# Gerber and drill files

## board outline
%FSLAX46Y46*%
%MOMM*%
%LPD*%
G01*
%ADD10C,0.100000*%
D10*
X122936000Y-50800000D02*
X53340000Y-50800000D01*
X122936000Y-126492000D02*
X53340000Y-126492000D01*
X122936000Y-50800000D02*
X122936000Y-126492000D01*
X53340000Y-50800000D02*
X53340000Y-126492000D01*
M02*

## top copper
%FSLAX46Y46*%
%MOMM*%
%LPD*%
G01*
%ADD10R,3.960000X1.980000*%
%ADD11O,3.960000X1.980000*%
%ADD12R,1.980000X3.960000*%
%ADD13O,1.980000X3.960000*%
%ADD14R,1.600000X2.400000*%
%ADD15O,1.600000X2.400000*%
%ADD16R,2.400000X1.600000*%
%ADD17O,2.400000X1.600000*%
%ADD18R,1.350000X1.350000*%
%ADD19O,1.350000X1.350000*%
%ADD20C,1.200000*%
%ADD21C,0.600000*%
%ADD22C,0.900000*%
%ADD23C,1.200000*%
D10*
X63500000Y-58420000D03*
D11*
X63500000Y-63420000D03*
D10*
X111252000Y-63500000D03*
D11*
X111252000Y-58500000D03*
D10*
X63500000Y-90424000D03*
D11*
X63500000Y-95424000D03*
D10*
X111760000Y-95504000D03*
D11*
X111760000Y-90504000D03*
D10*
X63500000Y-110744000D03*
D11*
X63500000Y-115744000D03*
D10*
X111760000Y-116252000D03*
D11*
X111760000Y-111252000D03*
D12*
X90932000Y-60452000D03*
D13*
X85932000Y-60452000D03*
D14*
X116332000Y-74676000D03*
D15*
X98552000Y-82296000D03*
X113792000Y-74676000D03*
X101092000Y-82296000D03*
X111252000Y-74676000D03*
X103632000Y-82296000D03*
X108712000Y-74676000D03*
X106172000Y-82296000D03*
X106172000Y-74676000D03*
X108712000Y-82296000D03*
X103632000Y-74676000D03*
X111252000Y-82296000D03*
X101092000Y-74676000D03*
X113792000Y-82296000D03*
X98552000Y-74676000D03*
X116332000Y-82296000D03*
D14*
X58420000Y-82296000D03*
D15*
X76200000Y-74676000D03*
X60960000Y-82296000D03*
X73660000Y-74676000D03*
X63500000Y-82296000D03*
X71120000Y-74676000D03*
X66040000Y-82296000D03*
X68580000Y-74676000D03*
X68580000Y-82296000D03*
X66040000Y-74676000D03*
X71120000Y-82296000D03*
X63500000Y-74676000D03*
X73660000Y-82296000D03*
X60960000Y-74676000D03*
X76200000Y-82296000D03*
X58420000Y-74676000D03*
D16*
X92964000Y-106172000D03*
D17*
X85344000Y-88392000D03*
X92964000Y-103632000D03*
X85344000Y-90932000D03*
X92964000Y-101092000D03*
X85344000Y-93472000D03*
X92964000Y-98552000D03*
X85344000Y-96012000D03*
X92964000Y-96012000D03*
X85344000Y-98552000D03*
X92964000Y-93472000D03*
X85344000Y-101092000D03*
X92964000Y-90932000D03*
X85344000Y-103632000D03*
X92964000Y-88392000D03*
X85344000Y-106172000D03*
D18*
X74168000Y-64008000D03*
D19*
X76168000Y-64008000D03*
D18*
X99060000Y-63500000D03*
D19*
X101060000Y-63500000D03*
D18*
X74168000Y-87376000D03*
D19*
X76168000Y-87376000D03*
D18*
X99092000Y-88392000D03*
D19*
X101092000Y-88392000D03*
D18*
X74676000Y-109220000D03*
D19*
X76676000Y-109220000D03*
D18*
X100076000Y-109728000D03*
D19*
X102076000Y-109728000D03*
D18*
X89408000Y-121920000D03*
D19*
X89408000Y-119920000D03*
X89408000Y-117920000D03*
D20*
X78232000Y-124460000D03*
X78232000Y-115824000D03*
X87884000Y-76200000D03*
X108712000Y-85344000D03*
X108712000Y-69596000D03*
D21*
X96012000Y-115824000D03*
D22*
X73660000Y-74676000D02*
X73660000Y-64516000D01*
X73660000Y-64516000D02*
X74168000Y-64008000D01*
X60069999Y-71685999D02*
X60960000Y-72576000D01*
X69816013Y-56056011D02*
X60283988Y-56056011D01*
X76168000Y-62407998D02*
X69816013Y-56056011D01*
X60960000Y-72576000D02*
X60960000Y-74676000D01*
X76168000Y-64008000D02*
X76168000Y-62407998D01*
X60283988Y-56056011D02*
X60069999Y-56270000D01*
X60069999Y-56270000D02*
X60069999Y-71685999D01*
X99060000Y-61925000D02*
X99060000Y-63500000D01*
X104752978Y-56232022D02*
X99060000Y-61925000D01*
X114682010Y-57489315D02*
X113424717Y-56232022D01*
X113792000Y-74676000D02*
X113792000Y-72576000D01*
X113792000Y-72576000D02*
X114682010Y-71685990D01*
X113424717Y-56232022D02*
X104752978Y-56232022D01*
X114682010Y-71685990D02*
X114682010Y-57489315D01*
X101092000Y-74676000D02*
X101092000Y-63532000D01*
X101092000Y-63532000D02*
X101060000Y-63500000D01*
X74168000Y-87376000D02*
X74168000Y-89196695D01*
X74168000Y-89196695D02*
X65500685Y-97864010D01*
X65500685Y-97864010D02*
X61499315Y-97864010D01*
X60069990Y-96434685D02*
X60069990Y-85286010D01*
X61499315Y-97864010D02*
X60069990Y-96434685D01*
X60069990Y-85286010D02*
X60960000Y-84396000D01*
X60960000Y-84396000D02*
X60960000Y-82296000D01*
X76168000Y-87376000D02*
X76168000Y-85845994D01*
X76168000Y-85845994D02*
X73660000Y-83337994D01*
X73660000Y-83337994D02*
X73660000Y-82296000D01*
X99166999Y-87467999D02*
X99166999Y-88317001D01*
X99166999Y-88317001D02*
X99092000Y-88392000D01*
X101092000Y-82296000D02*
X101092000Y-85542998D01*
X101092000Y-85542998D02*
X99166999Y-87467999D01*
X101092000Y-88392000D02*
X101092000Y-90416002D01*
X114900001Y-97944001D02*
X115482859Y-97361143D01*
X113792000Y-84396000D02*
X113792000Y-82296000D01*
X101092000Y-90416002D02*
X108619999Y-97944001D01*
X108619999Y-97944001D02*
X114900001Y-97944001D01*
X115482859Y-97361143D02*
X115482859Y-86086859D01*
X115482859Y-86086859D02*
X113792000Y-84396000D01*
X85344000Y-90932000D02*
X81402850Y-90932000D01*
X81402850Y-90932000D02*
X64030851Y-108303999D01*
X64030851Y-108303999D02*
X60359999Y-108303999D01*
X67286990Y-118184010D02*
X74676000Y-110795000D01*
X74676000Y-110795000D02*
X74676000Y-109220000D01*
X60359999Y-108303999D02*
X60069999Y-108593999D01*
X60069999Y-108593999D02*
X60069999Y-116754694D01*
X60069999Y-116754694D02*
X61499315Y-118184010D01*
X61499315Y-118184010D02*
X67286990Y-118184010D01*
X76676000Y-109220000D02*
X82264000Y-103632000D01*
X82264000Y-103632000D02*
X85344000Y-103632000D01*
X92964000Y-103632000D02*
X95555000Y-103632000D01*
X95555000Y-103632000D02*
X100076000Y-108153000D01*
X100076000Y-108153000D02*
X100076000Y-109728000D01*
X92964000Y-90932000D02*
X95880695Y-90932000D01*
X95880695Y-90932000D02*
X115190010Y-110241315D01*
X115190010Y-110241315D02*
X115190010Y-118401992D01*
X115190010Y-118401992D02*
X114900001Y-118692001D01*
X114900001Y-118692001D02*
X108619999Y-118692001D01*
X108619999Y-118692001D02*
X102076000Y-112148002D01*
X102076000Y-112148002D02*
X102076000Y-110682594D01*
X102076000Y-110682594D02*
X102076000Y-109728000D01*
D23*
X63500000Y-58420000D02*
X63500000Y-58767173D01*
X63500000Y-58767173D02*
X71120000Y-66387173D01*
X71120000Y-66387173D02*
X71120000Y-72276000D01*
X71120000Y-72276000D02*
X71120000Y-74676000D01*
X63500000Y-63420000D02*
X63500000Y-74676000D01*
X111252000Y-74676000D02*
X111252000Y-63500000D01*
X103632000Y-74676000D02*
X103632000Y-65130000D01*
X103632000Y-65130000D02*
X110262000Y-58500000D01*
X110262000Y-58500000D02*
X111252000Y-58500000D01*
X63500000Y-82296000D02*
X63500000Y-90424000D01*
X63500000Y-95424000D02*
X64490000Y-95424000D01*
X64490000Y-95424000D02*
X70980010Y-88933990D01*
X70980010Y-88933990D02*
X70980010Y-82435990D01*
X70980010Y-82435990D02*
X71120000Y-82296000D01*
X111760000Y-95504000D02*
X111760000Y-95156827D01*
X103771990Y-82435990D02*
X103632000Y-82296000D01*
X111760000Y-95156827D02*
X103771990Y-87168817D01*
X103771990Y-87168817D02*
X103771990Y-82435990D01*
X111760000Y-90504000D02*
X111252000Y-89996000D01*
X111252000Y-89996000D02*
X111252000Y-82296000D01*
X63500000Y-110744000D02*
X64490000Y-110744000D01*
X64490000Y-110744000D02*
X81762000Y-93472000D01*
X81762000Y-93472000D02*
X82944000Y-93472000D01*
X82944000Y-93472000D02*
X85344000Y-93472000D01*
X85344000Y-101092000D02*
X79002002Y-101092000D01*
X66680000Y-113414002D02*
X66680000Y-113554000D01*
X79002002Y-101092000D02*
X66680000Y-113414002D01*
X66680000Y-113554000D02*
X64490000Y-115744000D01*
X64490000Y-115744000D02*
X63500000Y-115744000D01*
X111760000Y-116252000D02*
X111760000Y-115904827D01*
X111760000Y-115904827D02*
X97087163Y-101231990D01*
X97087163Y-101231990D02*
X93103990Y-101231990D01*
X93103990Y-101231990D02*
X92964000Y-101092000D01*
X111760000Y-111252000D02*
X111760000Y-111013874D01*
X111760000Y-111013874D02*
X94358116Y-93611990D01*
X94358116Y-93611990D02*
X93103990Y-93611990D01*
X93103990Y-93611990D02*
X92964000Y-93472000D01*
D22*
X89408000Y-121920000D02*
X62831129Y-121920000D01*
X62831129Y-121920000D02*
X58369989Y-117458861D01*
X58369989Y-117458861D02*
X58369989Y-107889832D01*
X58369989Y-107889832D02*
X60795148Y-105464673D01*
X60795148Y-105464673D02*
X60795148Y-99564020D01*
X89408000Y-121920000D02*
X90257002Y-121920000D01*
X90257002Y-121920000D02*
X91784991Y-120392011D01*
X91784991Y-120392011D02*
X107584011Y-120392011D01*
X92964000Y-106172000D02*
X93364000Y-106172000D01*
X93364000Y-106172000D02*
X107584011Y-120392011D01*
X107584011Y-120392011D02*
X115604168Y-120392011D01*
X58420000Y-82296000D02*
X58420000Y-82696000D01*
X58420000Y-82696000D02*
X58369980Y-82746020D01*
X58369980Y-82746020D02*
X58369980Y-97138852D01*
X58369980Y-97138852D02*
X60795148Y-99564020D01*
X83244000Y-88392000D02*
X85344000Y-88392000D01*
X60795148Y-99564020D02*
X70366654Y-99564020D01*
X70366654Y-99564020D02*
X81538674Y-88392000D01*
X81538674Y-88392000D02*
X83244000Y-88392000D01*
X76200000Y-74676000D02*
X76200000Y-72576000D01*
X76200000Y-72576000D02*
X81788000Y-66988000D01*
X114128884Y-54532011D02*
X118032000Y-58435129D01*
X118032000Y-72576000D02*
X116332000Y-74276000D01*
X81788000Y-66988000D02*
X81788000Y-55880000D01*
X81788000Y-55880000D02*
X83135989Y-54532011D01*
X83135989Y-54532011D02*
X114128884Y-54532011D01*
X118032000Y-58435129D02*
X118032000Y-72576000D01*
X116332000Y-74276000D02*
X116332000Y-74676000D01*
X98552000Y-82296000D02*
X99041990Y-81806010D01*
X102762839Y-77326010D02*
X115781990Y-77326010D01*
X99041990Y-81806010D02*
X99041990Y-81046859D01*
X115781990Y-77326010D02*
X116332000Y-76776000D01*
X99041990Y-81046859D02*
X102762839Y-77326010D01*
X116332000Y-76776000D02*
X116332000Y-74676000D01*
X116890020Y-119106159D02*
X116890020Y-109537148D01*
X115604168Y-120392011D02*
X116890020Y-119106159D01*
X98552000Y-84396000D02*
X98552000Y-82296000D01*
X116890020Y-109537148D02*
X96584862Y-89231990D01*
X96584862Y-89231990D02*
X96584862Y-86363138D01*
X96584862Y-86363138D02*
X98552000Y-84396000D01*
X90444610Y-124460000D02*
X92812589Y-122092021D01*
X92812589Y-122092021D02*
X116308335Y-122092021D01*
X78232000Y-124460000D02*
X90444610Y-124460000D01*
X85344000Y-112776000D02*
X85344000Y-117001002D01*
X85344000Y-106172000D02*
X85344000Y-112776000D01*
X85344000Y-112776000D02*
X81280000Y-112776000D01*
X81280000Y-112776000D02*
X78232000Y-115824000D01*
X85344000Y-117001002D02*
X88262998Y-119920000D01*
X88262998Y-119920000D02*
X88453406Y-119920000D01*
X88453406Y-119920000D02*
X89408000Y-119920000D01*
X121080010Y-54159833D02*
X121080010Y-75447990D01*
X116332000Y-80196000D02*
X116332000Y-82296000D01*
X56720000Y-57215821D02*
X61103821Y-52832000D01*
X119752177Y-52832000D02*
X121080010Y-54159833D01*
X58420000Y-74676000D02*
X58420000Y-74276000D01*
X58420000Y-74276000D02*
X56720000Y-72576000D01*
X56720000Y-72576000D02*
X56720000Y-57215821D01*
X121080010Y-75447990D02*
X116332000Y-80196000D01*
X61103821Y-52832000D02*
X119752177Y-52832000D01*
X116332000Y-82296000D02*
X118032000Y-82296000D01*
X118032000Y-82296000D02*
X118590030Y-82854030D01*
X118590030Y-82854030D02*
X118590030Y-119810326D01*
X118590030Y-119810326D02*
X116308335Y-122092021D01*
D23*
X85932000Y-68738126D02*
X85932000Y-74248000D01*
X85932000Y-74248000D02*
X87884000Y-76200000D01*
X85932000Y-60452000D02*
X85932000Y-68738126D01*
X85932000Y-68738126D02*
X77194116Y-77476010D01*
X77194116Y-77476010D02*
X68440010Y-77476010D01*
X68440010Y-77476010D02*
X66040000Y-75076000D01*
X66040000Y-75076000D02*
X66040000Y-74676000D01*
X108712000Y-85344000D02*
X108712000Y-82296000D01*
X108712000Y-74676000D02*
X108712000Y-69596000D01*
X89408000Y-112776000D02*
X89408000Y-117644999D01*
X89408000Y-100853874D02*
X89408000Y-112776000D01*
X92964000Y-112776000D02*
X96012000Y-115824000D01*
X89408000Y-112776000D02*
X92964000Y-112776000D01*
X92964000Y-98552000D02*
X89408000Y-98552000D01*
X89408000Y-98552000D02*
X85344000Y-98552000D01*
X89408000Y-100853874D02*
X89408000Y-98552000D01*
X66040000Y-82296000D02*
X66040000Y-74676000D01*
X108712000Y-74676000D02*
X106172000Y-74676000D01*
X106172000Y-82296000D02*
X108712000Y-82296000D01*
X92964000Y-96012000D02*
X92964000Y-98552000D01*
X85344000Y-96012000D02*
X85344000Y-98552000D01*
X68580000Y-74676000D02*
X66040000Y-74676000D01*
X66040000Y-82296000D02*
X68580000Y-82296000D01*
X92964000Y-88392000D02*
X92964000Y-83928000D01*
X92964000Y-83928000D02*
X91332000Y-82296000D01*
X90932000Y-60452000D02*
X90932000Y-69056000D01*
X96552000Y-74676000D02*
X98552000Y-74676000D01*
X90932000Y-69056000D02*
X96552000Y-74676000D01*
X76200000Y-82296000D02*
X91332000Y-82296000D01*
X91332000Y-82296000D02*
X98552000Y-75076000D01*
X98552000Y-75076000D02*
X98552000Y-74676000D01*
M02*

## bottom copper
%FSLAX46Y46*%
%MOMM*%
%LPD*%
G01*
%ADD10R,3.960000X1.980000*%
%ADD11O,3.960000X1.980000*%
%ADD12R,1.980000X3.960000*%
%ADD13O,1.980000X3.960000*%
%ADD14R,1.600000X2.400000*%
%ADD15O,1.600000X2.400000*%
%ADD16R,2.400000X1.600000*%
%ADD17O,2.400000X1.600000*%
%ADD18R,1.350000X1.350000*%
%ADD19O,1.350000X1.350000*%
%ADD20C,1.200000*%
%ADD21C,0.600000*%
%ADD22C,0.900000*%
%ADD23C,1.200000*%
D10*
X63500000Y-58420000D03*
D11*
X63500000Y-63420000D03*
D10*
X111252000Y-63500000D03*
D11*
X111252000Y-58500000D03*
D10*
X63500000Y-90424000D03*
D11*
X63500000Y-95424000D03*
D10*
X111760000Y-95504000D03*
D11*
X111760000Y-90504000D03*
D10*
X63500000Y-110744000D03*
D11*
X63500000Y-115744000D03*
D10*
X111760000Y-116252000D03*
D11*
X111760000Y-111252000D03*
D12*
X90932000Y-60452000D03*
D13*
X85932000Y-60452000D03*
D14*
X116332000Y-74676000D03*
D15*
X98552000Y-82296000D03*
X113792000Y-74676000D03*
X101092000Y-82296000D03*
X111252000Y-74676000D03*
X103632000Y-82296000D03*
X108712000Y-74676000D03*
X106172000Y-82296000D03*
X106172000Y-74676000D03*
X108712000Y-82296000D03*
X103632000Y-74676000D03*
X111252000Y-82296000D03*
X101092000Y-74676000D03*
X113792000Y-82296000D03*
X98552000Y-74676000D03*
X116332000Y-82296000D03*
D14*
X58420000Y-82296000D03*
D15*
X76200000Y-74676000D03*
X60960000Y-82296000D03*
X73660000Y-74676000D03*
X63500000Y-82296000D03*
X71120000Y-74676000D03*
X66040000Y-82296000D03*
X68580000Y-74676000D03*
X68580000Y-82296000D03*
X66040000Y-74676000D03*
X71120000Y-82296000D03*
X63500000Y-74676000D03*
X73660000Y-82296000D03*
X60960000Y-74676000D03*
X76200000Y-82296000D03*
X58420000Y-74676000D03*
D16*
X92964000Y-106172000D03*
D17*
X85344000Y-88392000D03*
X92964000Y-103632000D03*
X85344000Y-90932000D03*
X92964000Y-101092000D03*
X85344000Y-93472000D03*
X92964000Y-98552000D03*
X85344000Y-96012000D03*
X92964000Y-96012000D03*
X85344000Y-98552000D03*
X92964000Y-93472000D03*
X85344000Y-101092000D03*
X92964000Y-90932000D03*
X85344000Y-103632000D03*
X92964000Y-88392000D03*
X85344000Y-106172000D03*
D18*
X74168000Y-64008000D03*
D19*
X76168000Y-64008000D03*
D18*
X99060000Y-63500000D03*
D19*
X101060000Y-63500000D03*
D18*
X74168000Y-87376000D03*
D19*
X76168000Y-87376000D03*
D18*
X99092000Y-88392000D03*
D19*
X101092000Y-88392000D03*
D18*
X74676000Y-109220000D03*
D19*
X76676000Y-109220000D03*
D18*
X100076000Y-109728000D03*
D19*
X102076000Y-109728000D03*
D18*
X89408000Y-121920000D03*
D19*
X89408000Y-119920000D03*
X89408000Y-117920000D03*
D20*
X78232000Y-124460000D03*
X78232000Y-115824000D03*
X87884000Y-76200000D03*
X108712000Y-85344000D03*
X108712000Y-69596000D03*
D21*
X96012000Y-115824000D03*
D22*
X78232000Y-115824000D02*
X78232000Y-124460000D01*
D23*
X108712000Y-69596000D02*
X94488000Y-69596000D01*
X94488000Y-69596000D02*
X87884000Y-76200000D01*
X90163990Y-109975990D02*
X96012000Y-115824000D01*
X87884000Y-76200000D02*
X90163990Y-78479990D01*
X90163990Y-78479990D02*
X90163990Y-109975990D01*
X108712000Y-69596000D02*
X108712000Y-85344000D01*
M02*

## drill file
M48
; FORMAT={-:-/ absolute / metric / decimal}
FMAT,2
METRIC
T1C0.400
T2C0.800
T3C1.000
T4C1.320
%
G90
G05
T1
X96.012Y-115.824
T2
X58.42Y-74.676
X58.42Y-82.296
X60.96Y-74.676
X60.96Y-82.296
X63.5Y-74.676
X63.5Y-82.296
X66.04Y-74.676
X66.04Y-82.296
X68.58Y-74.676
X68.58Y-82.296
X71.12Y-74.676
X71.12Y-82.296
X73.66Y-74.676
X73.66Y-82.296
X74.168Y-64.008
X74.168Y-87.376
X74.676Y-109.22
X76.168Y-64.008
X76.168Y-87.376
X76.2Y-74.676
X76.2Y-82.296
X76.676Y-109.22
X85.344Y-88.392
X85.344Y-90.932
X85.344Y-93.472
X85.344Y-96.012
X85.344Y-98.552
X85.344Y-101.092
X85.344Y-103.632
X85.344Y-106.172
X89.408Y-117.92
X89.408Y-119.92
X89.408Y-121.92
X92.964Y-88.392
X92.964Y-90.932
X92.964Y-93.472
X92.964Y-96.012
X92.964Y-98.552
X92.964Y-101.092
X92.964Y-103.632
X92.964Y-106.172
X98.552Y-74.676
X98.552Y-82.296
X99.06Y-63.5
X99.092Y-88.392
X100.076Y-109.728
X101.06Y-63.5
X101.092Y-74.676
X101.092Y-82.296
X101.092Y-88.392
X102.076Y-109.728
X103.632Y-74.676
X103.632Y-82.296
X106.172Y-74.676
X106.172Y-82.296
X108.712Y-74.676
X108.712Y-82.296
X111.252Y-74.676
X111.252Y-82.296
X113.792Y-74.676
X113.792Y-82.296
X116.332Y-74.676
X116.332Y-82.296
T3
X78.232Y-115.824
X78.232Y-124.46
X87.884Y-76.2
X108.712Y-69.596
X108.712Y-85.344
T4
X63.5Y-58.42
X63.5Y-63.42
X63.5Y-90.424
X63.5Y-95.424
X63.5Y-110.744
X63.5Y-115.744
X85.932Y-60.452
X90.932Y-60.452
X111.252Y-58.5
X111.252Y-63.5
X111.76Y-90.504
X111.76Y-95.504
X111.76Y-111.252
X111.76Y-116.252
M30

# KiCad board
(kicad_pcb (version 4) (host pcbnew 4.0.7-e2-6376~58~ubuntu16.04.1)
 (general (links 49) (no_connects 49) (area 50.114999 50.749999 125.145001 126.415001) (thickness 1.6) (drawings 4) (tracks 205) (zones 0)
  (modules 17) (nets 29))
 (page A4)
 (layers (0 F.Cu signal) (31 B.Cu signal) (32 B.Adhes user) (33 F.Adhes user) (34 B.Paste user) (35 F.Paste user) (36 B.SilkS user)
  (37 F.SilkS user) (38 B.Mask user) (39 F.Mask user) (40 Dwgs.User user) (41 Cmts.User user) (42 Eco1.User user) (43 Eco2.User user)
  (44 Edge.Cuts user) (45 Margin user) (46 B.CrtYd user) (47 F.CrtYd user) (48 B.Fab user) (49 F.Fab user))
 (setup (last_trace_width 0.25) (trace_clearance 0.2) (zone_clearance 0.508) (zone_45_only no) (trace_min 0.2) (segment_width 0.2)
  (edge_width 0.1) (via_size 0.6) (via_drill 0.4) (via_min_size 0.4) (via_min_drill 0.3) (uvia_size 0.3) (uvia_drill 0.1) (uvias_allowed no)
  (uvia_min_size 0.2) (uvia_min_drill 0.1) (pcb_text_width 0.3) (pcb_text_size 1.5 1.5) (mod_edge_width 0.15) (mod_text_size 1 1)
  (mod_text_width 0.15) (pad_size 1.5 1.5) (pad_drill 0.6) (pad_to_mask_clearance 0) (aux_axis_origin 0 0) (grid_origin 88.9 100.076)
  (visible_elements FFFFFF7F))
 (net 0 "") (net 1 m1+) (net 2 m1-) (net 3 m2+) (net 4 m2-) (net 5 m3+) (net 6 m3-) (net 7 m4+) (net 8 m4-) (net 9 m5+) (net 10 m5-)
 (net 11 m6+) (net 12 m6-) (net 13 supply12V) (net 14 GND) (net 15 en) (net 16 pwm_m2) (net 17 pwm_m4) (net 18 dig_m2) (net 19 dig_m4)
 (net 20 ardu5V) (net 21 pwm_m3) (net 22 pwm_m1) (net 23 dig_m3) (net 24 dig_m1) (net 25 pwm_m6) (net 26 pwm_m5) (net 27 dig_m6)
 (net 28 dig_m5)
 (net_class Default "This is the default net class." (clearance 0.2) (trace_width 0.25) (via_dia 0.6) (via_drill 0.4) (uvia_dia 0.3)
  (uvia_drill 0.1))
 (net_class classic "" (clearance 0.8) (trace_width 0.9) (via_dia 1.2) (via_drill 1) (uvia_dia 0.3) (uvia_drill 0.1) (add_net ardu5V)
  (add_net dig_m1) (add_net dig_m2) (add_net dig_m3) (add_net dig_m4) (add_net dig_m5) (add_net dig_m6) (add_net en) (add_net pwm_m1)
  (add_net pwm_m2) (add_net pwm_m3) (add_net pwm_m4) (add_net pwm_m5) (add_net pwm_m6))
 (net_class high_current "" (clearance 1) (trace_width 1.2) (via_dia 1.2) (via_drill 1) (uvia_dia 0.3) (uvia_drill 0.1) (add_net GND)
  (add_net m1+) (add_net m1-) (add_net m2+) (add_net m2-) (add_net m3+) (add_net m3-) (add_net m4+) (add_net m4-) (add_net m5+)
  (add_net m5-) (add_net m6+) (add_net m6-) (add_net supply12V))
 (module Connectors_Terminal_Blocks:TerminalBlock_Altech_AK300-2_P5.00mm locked (layer F.Cu) (at 63.5 58.42 270)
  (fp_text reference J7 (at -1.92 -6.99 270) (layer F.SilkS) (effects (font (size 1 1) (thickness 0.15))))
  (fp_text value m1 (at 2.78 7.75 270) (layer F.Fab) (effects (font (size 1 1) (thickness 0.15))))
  (pad 1 thru_hole rect (at 0 0 270) (size 1.98 3.96) (drill 1.32) (layers *.Cu *.Mask) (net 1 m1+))
  (pad 2 thru_hole oval (at 5 0 270) (size 1.98 3.96) (drill 1.32) (layers *.Cu *.Mask) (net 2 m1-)))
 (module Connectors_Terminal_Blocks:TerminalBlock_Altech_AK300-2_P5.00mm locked (layer F.Cu) (at 111.252 63.5 90)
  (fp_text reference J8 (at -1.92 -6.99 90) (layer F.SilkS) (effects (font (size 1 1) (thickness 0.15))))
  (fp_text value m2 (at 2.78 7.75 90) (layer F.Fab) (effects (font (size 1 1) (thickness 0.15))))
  (pad 1 thru_hole rect (at 0 0 90) (size 1.98 3.96) (drill 1.32) (layers *.Cu *.Mask) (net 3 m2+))
  (pad 2 thru_hole oval (at 5 0 90) (size 1.98 3.96) (drill 1.32) (layers *.Cu *.Mask) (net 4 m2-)))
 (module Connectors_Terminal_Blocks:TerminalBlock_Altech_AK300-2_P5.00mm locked (layer F.Cu) (at 63.5 90.424 270)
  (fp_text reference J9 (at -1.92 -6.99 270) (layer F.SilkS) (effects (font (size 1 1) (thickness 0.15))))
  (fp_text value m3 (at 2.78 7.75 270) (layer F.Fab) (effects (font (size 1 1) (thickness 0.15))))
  (pad 1 thru_hole rect (at 0 0 270) (size 1.98 3.96) (drill 1.32) (layers *.Cu *.Mask) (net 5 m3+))
  (pad 2 thru_hole oval (at 5 0 270) (size 1.98 3.96) (drill 1.32) (layers *.Cu *.Mask) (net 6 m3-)))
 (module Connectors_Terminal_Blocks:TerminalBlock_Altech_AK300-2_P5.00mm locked (layer F.Cu) (at 111.76 95.504 90)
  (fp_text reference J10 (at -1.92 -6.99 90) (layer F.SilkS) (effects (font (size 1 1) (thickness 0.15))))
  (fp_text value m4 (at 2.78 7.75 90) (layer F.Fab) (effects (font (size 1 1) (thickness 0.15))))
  (pad 1 thru_hole rect (at 0 0 90) (size 1.98 3.96) (drill 1.32) (layers *.Cu *.Mask) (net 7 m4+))
  (pad 2 thru_hole oval (at 5 0 90) (size 1.98 3.96) (drill 1.32) (layers *.Cu *.Mask) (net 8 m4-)))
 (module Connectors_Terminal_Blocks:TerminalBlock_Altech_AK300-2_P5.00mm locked (layer F.Cu) (at 63.5 110.744 270)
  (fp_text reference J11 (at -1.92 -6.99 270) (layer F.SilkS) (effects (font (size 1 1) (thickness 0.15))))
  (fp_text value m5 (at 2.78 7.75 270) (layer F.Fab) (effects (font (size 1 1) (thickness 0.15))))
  (pad 1 thru_hole rect (at 0 0 270) (size 1.98 3.96) (drill 1.32) (layers *.Cu *.Mask) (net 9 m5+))
  (pad 2 thru_hole oval (at 5 0 270) (size 1.98 3.96) (drill 1.32) (layers *.Cu *.Mask) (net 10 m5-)))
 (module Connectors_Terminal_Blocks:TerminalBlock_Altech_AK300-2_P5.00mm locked (layer F.Cu) (at 111.76 116.252 90)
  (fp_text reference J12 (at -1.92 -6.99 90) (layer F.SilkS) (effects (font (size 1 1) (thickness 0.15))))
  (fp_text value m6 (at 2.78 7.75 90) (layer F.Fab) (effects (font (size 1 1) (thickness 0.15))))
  (pad 1 thru_hole rect (at 0 0 90) (size 1.98 3.96) (drill 1.32) (layers *.Cu *.Mask) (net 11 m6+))
  (pad 2 thru_hole oval (at 5 0 90) (size 1.98 3.96) (drill 1.32) (layers *.Cu *.Mask) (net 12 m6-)))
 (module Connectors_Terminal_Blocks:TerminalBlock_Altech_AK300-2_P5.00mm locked (layer F.Cu) (at 90.932 60.452 180)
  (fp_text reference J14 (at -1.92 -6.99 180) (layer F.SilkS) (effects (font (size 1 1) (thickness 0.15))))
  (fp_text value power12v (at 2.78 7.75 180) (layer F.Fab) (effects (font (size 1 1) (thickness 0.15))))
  (pad 1 thru_hole rect (at 0 0 180) (size 1.98 3.96) (drill 1.32) (layers *.Cu *.Mask) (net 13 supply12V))
  (pad 2 thru_hole oval (at 5 0 180) (size 1.98 3.96) (drill 1.32) (layers *.Cu *.Mask) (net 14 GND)))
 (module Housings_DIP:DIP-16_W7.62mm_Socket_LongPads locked (layer F.Cu) (at 116.332 74.676 270)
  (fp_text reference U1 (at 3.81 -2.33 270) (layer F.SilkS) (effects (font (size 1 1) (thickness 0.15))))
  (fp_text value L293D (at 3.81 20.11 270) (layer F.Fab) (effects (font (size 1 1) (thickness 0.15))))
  (pad 1 thru_hole rect (at 0 0 270) (size 2.4 1.6) (drill 0.8) (layers *.Cu *.Mask) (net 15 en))
  (pad 9 thru_hole oval (at 7.62 17.78 270) (size 2.4 1.6) (drill 0.8) (layers *.Cu *.Mask) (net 15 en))
  (pad 2 thru_hole oval (at 0 2.54 270) (size 2.4 1.6) (drill 0.8) (layers *.Cu *.Mask) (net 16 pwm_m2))
  (pad 10 thru_hole oval (at 7.62 15.24 270) (size 2.4 1.6) (drill 0.8) (layers *.Cu *.Mask) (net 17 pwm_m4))
  (pad 3 thru_hole oval (at 0 5.08 270) (size 2.4 1.6) (drill 0.8) (layers *.Cu *.Mask) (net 3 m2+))
  (pad 11 thru_hole oval (at 7.62 12.7 270) (size 2.4 1.6) (drill 0.8) (layers *.Cu *.Mask) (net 7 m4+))
  (pad 4 thru_hole oval (at 0 7.62 270) (size 2.4 1.6) (drill 0.8) (layers *.Cu *.Mask) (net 14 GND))
  (pad 12 thru_hole oval (at 7.62 10.16 270) (size 2.4 1.6) (drill 0.8) (layers *.Cu *.Mask) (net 14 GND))
  (pad 5 thru_hole oval (at 0 10.16 270) (size 2.4 1.6) (drill 0.8) (layers *.Cu *.Mask) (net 14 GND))
  (pad 13 thru_hole oval (at 7.62 7.62 270) (size 2.4 1.6) (drill 0.8) (layers *.Cu *.Mask) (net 14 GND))
  (pad 6 thru_hole oval (at 0 12.7 270) (size 2.4 1.6) (drill 0.8) (layers *.Cu *.Mask) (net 4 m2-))
  (pad 14 thru_hole oval (at 7.62 5.08 270) (size 2.4 1.6) (drill 0.8) (layers *.Cu *.Mask) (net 8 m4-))
  (pad 7 thru_hole oval (at 0 15.24 270) (size 2.4 1.6) (drill 0.8) (layers *.Cu *.Mask) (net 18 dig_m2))
  (pad 15 thru_hole oval (at 7.62 2.54 270) (size 2.4 1.6) (drill 0.8) (layers *.Cu *.Mask) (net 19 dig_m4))
  (pad 8 thru_hole oval (at 0 17.78 270) (size 2.4 1.6) (drill 0.8) (layers *.Cu *.Mask) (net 13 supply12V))
  (pad 16 thru_hole oval (at 7.62 0 270) (size 2.4 1.6) (drill 0.8) (layers *.Cu *.Mask) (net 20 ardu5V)))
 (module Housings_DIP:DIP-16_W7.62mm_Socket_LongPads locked (layer F.Cu) (at 58.42 82.296 90)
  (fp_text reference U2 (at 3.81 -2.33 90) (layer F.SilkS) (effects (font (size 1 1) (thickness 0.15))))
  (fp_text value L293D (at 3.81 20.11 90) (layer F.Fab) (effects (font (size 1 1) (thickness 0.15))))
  (pad 1 thru_hole rect (at 0 0 90) (size 2.4 1.6) (drill 0.8) (layers *.Cu *.Mask) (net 15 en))
  (pad 9 thru_hole oval (at 7.62 17.78 90) (size 2.4 1.6) (drill 0.8) (layers *.Cu *.Mask) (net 15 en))
  (pad 2 thru_hole oval (at 0 2.54 90) (size 2.4 1.6) (drill 0.8) (layers *.Cu *.Mask) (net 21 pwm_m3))
  (pad 10 thru_hole oval (at 7.62 15.24 90) (size 2.4 1.6) (drill 0.8) (layers *.Cu *.Mask) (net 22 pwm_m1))
  (pad 3 thru_hole oval (at 0 5.08 90) (size 2.4 1.6) (drill 0.8) (layers *.Cu *.Mask) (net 5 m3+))
  (pad 11 thru_hole oval (at 7.62 12.7 90) (size 2.4 1.6) (drill 0.8) (layers *.Cu *.Mask) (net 1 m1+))
  (pad 4 thru_hole oval (at 0 7.62 90) (size 2.4 1.6) (drill 0.8) (layers *.Cu *.Mask) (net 14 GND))
  (pad 12 thru_hole oval (at 7.62 10.16 90) (size 2.4 1.6) (drill 0.8) (layers *.Cu *.Mask) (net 14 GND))
  (pad 5 thru_hole oval (at 0 10.16 90) (size 2.4 1.6) (drill 0.8) (layers *.Cu *.Mask) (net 14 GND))
  (pad 13 thru_hole oval (at 7.62 7.62 90) (size 2.4 1.6) (drill 0.8) (layers *.Cu *.Mask) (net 14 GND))
  (pad 6 thru_hole oval (at 0 12.7 90) (size 2.4 1.6) (drill 0.8) (layers *.Cu *.Mask) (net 6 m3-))
  (pad 14 thru_hole oval (at 7.62 5.08 90) (size 2.4 1.6) (drill 0.8) (layers *.Cu *.Mask) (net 2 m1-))
  (pad 7 thru_hole oval (at 0 15.24 90) (size 2.4 1.6) (drill 0.8) (layers *.Cu *.Mask) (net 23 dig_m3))
  (pad 15 thru_hole oval (at 7.62 2.54 90) (size 2.4 1.6) (drill 0.8) (layers *.Cu *.Mask) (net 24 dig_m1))
  (pad 8 thru_hole oval (at 0 17.78 90) (size 2.4 1.6) (drill 0.8) (layers *.Cu *.Mask) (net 13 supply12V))
  (pad 16 thru_hole oval (at 7.62 0 90) (size 2.4 1.6) (drill 0.8) (layers *.Cu *.Mask) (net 20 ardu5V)))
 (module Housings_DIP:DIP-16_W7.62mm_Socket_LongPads (layer F.Cu) (at 92.964 106.172 180)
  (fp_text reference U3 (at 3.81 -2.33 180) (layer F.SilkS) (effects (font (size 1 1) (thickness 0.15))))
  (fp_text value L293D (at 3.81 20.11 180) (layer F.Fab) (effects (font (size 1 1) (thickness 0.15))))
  (pad 1 thru_hole rect (at 0 0 180) (size 2.4 1.6) (drill 0.8) (layers *.Cu *.Mask) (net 15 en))
  (pad 9 thru_hole oval (at 7.62 17.78 180) (size 2.4 1.6) (drill 0.8) (layers *.Cu *.Mask) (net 15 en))
  (pad 2 thru_hole oval (at 0 2.54 180) (size 2.4 1.6) (drill 0.8) (layers *.Cu *.Mask) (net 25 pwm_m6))
  (pad 10 thru_hole oval (at 7.62 15.24 180) (size 2.4 1.6) (drill 0.8) (layers *.Cu *.Mask) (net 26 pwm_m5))
  (pad 3 thru_hole oval (at 0 5.08 180) (size 2.4 1.6) (drill 0.8) (layers *.Cu *.Mask) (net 11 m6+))
  (pad 11 thru_hole oval (at 7.62 12.7 180) (size 2.4 1.6) (drill 0.8) (layers *.Cu *.Mask) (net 9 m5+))
  (pad 4 thru_hole oval (at 0 7.62 180) (size 2.4 1.6) (drill 0.8) (layers *.Cu *.Mask) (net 14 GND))
  (pad 12 thru_hole oval (at 7.62 10.16 180) (size 2.4 1.6) (drill 0.8) (layers *.Cu *.Mask) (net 14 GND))
  (pad 5 thru_hole oval (at 0 10.16 180) (size 2.4 1.6) (drill 0.8) (layers *.Cu *.Mask) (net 14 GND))
  (pad 13 thru_hole oval (at 7.62 7.62 180) (size 2.4 1.6) (drill 0.8) (layers *.Cu *.Mask) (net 14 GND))
  (pad 6 thru_hole oval (at 0 12.7 180) (size 2.4 1.6) (drill 0.8) (layers *.Cu *.Mask) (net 12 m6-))
  (pad 14 thru_hole oval (at 7.62 5.08 180) (size 2.4 1.6) (drill 0.8) (layers *.Cu *.Mask) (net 10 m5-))
  (pad 7 thru_hole oval (at 0 15.24 180) (size 2.4 1.6) (drill 0.8) (layers *.Cu *.Mask) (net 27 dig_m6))
  (pad 15 thru_hole oval (at 7.62 2.54 180) (size 2.4 1.6) (drill 0.8) (layers *.Cu *.Mask) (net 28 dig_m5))
  (pad 8 thru_hole oval (at 0 17.78 180) (size 2.4 1.6) (drill 0.8) (layers *.Cu *.Mask) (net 13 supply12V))
  (pad 16 thru_hole oval (at 7.62 0 180) (size 2.4 1.6) (drill 0.8) (layers *.Cu *.Mask) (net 20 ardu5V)))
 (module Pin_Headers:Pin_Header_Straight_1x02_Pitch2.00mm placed (layer F.Cu) (at 74.168 64.008 90)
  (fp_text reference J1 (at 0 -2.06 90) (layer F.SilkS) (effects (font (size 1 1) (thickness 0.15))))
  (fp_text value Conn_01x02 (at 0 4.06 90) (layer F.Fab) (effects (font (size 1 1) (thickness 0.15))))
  (pad 1 thru_hole rect (at 0 0 90) (size 1.35 1.35) (drill 0.8) (layers *.Cu *.Mask) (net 22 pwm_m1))
  (pad 2 thru_hole oval (at 0 2 90) (size 1.35 1.35) (drill 0.8) (layers *.Cu *.Mask) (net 24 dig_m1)))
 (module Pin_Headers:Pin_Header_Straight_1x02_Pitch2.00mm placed (layer F.Cu) (at 99.06 63.5 90)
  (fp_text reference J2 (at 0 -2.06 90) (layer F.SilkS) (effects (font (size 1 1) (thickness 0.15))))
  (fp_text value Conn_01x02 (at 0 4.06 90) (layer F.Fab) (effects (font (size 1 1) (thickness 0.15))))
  (pad 1 thru_hole rect (at 0 0 90) (size 1.35 1.35) (drill 0.8) (layers *.Cu *.Mask) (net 16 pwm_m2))
  (pad 2 thru_hole oval (at 0 2 90) (size 1.35 1.35) (drill 0.8) (layers *.Cu *.Mask) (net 18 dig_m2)))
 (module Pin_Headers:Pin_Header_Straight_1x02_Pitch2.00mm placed (layer F.Cu) (at 74.168 87.376 90)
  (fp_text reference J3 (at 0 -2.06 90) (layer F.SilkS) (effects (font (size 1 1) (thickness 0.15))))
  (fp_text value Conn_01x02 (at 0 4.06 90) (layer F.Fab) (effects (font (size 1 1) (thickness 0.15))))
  (pad 1 thru_hole rect (at 0 0 90) (size 1.35 1.35) (drill 0.8) (layers *.Cu *.Mask) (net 21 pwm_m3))
  (pad 2 thru_hole oval (at 0 2 90) (size 1.35 1.35) (drill 0.8) (layers *.Cu *.Mask) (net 23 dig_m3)))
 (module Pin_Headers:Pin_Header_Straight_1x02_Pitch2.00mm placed (layer F.Cu) (at 99.092 88.392 90)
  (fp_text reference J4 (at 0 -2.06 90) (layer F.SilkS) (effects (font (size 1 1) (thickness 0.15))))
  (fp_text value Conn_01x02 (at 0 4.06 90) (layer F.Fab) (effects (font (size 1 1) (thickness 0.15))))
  (pad 1 thru_hole rect (at 0 0 90) (size 1.35 1.35) (drill 0.8) (layers *.Cu *.Mask) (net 17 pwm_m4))
  (pad 2 thru_hole oval (at 0 2 90) (size 1.35 1.35) (drill 0.8) (layers *.Cu *.Mask) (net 19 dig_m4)))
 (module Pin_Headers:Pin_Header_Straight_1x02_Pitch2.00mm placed (layer F.Cu) (at 74.676 109.22 90)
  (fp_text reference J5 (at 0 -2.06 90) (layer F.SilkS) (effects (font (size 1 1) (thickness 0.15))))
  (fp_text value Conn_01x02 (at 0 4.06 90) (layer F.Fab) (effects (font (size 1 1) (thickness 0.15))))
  (pad 1 thru_hole rect (at 0 0 90) (size 1.35 1.35) (drill 0.8) (layers *.Cu *.Mask) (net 26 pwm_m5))
  (pad 2 thru_hole oval (at 0 2 90) (size 1.35 1.35) (drill 0.8) (layers *.Cu *.Mask) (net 28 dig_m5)))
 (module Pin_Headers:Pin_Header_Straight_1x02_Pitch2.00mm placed (layer F.Cu) (at 100.076 109.728 90)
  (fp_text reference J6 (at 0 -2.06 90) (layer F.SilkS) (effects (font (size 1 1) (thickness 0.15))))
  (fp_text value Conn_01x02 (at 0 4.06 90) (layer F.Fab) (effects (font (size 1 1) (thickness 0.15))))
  (pad 1 thru_hole rect (at 0 0 90) (size 1.35 1.35) (drill 0.8) (layers *.Cu *.Mask) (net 25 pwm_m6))
  (pad 2 thru_hole oval (at 0 2 90) (size 1.35 1.35) (drill 0.8) (layers *.Cu *.Mask) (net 27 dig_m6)))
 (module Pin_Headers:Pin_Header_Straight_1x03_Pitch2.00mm (layer F.Cu) (at 89.408 121.92 180)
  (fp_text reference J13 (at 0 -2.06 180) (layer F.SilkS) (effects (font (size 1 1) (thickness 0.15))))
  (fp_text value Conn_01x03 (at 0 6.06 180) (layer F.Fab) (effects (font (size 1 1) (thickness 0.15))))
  (pad 1 thru_hole rect (at 0 0 180) (size 1.35 1.35) (drill 0.8) (layers *.Cu *.Mask) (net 15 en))
  (pad 2 thru_hole oval (at 0 2 180) (size 1.35 1.35) (drill 0.8) (layers *.Cu *.Mask) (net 20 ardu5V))
  (pad 3 thru_hole oval (at 0 4 180) (size 1.35 1.35) (drill 0.8) (layers *.Cu *.Mask) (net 14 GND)))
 (gr_line (start 122.936 50.8) (end 53.34 50.8) (layer Edge.Cuts) (width 0.1))
 (gr_line (start 122.936 126.492) (end 53.34 126.492) (layer Edge.Cuts) (width 0.1))
 (gr_line (start 122.936 50.8) (end 122.936 126.492) (layer Edge.Cuts) (width 0.1))
 (gr_line (start 53.34 50.8) (end 53.34 126.492) (layer Edge.Cuts) (width 0.1))
 (segment (start 73.66 74.676) (end 73.66 64.516) (width 0.9) (layer F.Cu) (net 22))
 (segment (start 73.66 64.516) (end 74.168 64.008) (width 0.9) (layer F.Cu) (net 22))
 (segment (start 60.069999 71.685999) (end 60.96 72.576) (width 0.9) (layer F.Cu) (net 24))
 (segment (start 69.816013 56.056011) (end 60.283988 56.056011) (width 0.9) (layer F.Cu) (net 24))
 (segment (start 76.168 62.407998) (end 69.816013 56.056011) (width 0.9) (layer F.Cu) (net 24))
 (segment (start 60.96 72.576) (end 60.96 74.676) (width 0.9) (layer F.Cu) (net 24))
 (segment (start 76.168 64.008) (end 76.168 62.407998) (width 0.9) (layer F.Cu) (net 24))
 (segment (start 60.283988 56.056011) (end 60.069999 56.27) (width 0.9) (layer F.Cu) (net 24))
 (segment (start 60.069999 56.27) (end 60.069999 71.685999) (width 0.9) (layer F.Cu) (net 24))
 (segment (start 99.06 61.925) (end 99.06 63.5) (width 0.9) (layer F.Cu) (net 16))
 (segment (start 104.752978 56.232022) (end 99.06 61.925) (width 0.9) (layer F.Cu) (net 16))
 (segment (start 114.68201 57.489315) (end 113.424717 56.232022) (width 0.9) (layer F.Cu) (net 16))
 (segment (start 113.792 74.676) (end 113.792 72.576) (width 0.9) (layer F.Cu) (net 16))
 (segment (start 113.792 72.576) (end 114.68201 71.68599) (width 0.9) (layer F.Cu) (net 16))
 (segment (start 113.424717 56.232022) (end 104.752978 56.232022) (width 0.9) (layer F.Cu) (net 16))
 (segment (start 114.68201 71.68599) (end 114.68201 57.489315) (width 0.9) (layer F.Cu) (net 16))
 (segment (start 101.092 74.676) (end 101.092 63.532) (width 0.9) (layer F.Cu) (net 18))
 (segment (start 101.092 63.532) (end 101.06 63.5) (width 0.9) (layer F.Cu) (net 18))
 (segment (start 74.168 87.376) (end 74.168 89.196695) (width 0.9) (layer F.Cu) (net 21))
 (segment (start 74.168 89.196695) (end 65.500685 97.86401) (width 0.9) (layer F.Cu) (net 21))
 (segment (start 65.500685 97.86401) (end 61.499315 97.86401) (width 0.9) (layer F.Cu) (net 21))
 (segment (start 60.06999 96.434685) (end 60.06999 85.28601) (width 0.9) (layer F.Cu) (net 21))
 (segment (start 61.499315 97.86401) (end 60.06999 96.434685) (width 0.9) (layer F.Cu) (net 21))
 (segment (start 60.06999 85.28601) (end 60.96 84.396) (width 0.9) (layer F.Cu) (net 21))
 (segment (start 60.96 84.396) (end 60.96 82.296) (width 0.9) (layer F.Cu) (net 21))
 (segment (start 76.168 87.376) (end 76.168 85.845994) (width 0.9) (layer F.Cu) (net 23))
 (segment (start 76.168 85.845994) (end 73.66 83.337994) (width 0.9) (layer F.Cu) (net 23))
 (segment (start 73.66 83.337994) (end 73.66 82.296) (width 0.9) (layer F.Cu) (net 23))
 (segment (start 99.166999 87.467999) (end 99.166999 88.317001) (width 0.9) (layer F.Cu) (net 17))
 (segment (start 99.166999 88.317001) (end 99.092 88.392) (width 0.9) (layer F.Cu) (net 17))
 (segment (start 101.092 82.296) (end 101.092 85.542998) (width 0.9) (layer F.Cu) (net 17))
 (segment (start 101.092 85.542998) (end 99.166999 87.467999) (width 0.9) (layer F.Cu) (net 17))
 (segment (start 101.092 88.392) (end 101.092 90.416002) (width 0.9) (layer F.Cu) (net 19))
 (segment (start 114.900001 97.944001) (end 115.482859 97.361143) (width 0.9) (layer F.Cu) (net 19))
 (segment (start 113.792 84.396) (end 113.792 82.296) (width 0.9) (layer F.Cu) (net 19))
 (segment (start 101.092 90.416002) (end 108.619999 97.944001) (width 0.9) (layer F.Cu) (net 19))
 (segment (start 108.619999 97.944001) (end 114.900001 97.944001) (width 0.9) (layer F.Cu) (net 19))
 (segment (start 115.482859 97.361143) (end 115.482859 86.086859) (width 0.9) (layer F.Cu) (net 19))
 (segment (start 115.482859 86.086859) (end 113.792 84.396) (width 0.9) (layer F.Cu) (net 19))
 (segment (start 85.344 90.932) (end 81.40285 90.932) (width 0.9) (layer F.Cu) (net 26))
 (segment (start 81.40285 90.932) (end 64.030851 108.303999) (width 0.9) (layer F.Cu) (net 26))
 (segment (start 64.030851 108.303999) (end 60.359999 108.303999) (width 0.9) (layer F.Cu) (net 26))
 (segment (start 67.28699 118.18401) (end 74.676 110.795) (width 0.9) (layer F.Cu) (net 26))
 (segment (start 74.676 110.795) (end 74.676 109.22) (width 0.9) (layer F.Cu) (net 26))
 (segment (start 60.359999 108.303999) (end 60.069999 108.593999) (width 0.9) (layer F.Cu) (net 26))
 (segment (start 60.069999 108.593999) (end 60.069999 116.754694) (width 0.9) (layer F.Cu) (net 26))
 (segment (start 60.069999 116.754694) (end 61.499315 118.18401) (width 0.9) (layer F.Cu) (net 26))
 (segment (start 61.499315 118.18401) (end 67.28699 118.18401) (width 0.9) (layer F.Cu) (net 26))
 (segment (start 76.676 109.22) (end 82.264 103.632) (width 0.9) (layer F.Cu) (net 28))
 (segment (start 82.264 103.632) (end 85.344 103.632) (width 0.9) (layer F.Cu) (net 28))
 (segment (start 92.964 103.632) (end 95.555 103.632) (width 0.9) (layer F.Cu) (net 25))
 (segment (start 95.555 103.632) (end 100.076 108.153) (width 0.9) (layer F.Cu) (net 25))
 (segment (start 100.076 108.153) (end 100.076 109.728) (width 0.9) (layer F.Cu) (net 25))
 (segment (start 92.964 90.932) (end 95.880695 90.932) (width 0.9) (layer F.Cu) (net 27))
 (segment (start 95.880695 90.932) (end 115.19001 110.241315) (width 0.9) (layer F.Cu) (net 27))
 (segment (start 115.19001 110.241315) (end 115.19001 118.401992) (width 0.9) (layer F.Cu) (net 27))
 (segment (start 115.19001 118.401992) (end 114.900001 118.692001) (width 0.9) (layer F.Cu) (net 27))
 (segment (start 114.900001 118.692001) (end 108.619999 118.692001) (width 0.9) (layer F.Cu) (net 27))
 (segment (start 108.619999 118.692001) (end 102.076 112.148002) (width 0.9) (layer F.Cu) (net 27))
 (segment (start 102.076 112.148002) (end 102.076 110.682594) (width 0.9) (layer F.Cu) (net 27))
 (segment (start 102.076 110.682594) (end 102.076 109.728) (width 0.9) (layer F.Cu) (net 27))
 (segment (start 63.5 58.42) (end 63.5 58.767173) (width 1.2) (layer F.Cu) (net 1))
 (segment (start 63.5 58.767173) (end 71.12 66.387173) (width 1.2) (layer F.Cu) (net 1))
 (segment (start 71.12 66.387173) (end 71.12 72.276) (width 1.2) (layer F.Cu) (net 1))
 (segment (start 71.12 72.276) (end 71.12 74.676) (width 1.2) (layer F.Cu) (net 1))
 (segment (start 63.5 63.42) (end 63.5 74.676) (width 1.2) (layer F.Cu) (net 2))
 (segment (start 111.252 74.676) (end 111.252 63.5) (width 1.2) (layer F.Cu) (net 3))
 (segment (start 103.632 74.676) (end 103.632 65.13) (width 1.2) (layer F.Cu) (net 4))
 (segment (start 103.632 65.13) (end 110.262 58.5) (width 1.2) (layer F.Cu) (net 4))
 (segment (start 110.262 58.5) (end 111.252 58.5) (width 1.2) (layer F.Cu) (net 4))
 (segment (start 63.5 82.296) (end 63.5 90.424) (width 1.2) (layer F.Cu) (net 5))
 (segment (start 63.5 95.424) (end 64.49 95.424) (width 1.2) (layer F.Cu) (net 6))
 (segment (start 64.49 95.424) (end 70.98001 88.93399) (width 1.2) (layer F.Cu) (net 6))
 (segment (start 70.98001 88.93399) (end 70.98001 82.43599) (width 1.2) (layer F.Cu) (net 6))
 (segment (start 70.98001 82.43599) (end 71.12 82.296) (width 1.2) (layer F.Cu) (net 6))
 (segment (start 111.76 95.504) (end 111.76 95.156827) (width 1.2) (layer F.Cu) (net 7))
 (segment (start 103.77199 82.43599) (end 103.632 82.296) (width 1.2) (layer F.Cu) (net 7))
 (segment (start 111.76 95.156827) (end 103.77199 87.168817) (width 1.2) (layer F.Cu) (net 7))
 (segment (start 103.77199 87.168817) (end 103.77199 82.43599) (width 1.2) (layer F.Cu) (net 7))
 (segment (start 111.76 90.504) (end 111.252 89.996) (width 1.2) (layer F.Cu) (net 8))
 (segment (start 111.252 89.996) (end 111.252 82.296) (width 1.2) (layer F.Cu) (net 8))
 (segment (start 63.5 110.744) (end 64.49 110.744) (width 1.2) (layer F.Cu) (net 9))
 (segment (start 64.49 110.744) (end 81.762 93.472) (width 1.2) (layer F.Cu) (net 9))
 (segment (start 81.762 93.472) (end 82.944 93.472) (width 1.2) (layer F.Cu) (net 9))
 (segment (start 82.944 93.472) (end 85.344 93.472) (width 1.2) (layer F.Cu) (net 9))
 (segment (start 85.344 101.092) (end 79.002002 101.092) (width 1.2) (layer F.Cu) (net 10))
 (segment (start 66.68 113.414002) (end 66.68 113.554) (width 1.2) (layer F.Cu) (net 10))
 (segment (start 79.002002 101.092) (end 66.68 113.414002) (width 1.2) (layer F.Cu) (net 10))
 (segment (start 66.68 113.554) (end 64.49 115.744) (width 1.2) (layer F.Cu) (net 10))
 (segment (start 64.49 115.744) (end 63.5 115.744) (width 1.2) (layer F.Cu) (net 10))
 (segment (start 111.76 116.252) (end 111.76 115.904827) (width 1.2) (layer F.Cu) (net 11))
 (segment (start 111.76 115.904827) (end 97.087163 101.23199) (width 1.2) (layer F.Cu) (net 11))
 (segment (start 97.087163 101.23199) (end 93.10399 101.23199) (width 1.2) (layer F.Cu) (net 11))
 (segment (start 93.10399 101.23199) (end 92.964 101.092) (width 1.2) (layer F.Cu) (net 11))
 (segment (start 111.76 111.252) (end 111.76 111.013874) (width 1.2) (layer F.Cu) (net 12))
 (segment (start 111.76 111.013874) (end 94.358116 93.61199) (width 1.2) (layer F.Cu) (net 12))
 (segment (start 94.358116 93.61199) (end 93.10399 93.61199) (width 1.2) (layer F.Cu) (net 12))
 (segment (start 93.10399 93.61199) (end 92.964 93.472) (width 1.2) (layer F.Cu) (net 12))
 (segment (start 89.408 121.92) (end 62.831129 121.92) (width 0.9) (layer F.Cu) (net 15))
 (segment (start 62.831129 121.92) (end 58.369989 117.458861) (width 0.9) (layer F.Cu) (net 15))
 (segment (start 58.369989 117.458861) (end 58.369989 107.889832) (width 0.9) (layer F.Cu) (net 15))
 (segment (start 58.369989 107.889832) (end 60.795148 105.464673) (width 0.9) (layer F.Cu) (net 15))
 (segment (start 60.795148 105.464673) (end 60.795148 99.56402) (width 0.9) (layer F.Cu) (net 15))
 (segment (start 89.408 121.92) (end 90.257002 121.92) (width 0.9) (layer F.Cu) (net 15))
 (segment (start 90.257002 121.92) (end 91.784991 120.392011) (width 0.9) (layer F.Cu) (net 15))
 (segment (start 91.784991 120.392011) (end 107.584011 120.392011) (width 0.9) (layer F.Cu) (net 15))
 (segment (start 92.964 106.172) (end 93.364 106.172) (width 0.9) (layer F.Cu) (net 15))
 (segment (start 93.364 106.172) (end 107.584011 120.392011) (width 0.9) (layer F.Cu) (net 15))
 (segment (start 107.584011 120.392011) (end 115.604168 120.392011) (width 0.9) (layer F.Cu) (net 15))
 (segment (start 58.42 82.296) (end 58.42 82.696) (width 0.9) (layer F.Cu) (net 15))
 (segment (start 58.42 82.696) (end 58.36998 82.74602) (width 0.9) (layer F.Cu) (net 15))
 (segment (start 58.36998 82.74602) (end 58.36998 97.138852) (width 0.9) (layer F.Cu) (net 15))
 (segment (start 58.36998 97.138852) (end 60.795148 99.56402) (width 0.9) (layer F.Cu) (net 15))
 (segment (start 83.244 88.392) (end 85.344 88.392) (width 0.9) (layer F.Cu) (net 15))
 (segment (start 60.795148 99.56402) (end 70.366654 99.56402) (width 0.9) (layer F.Cu) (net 15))
 (segment (start 70.366654 99.56402) (end 81.538674 88.392) (width 0.9) (layer F.Cu) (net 15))
 (segment (start 81.538674 88.392) (end 83.244 88.392) (width 0.9) (layer F.Cu) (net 15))
 (segment (start 76.2 74.676) (end 76.2 72.576) (width 0.9) (layer F.Cu) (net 15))
 (segment (start 76.2 72.576) (end 81.788 66.988) (width 0.9) (layer F.Cu) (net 15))
 (segment (start 114.128884 54.532011) (end 118.032 58.435129) (width 0.9) (layer F.Cu) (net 15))
 (segment (start 118.032 72.576) (end 116.332 74.276) (width 0.9) (layer F.Cu) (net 15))
 (segment (start 81.788 66.988) (end 81.788 55.88) (width 0.9) (layer F.Cu) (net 15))
 (segment (start 81.788 55.88) (end 83.135989 54.532011) (width 0.9) (layer F.Cu) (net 15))
 (segment (start 83.135989 54.532011) (end 114.128884 54.532011) (width 0.9) (layer F.Cu) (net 15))
 (segment (start 118.032 58.435129) (end 118.032 72.576) (width 0.9) (layer F.Cu) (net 15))
 (segment (start 116.332 74.276) (end 116.332 74.676) (width 0.9) (layer F.Cu) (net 15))
 (segment (start 98.552 82.296) (end 99.04199 81.80601) (width 0.9) (layer F.Cu) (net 15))
 (segment (start 102.762839 77.32601) (end 115.78199 77.32601) (width 0.9) (layer F.Cu) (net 15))
 (segment (start 99.04199 81.80601) (end 99.04199 81.046859) (width 0.9) (layer F.Cu) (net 15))
 (segment (start 115.78199 77.32601) (end 116.332 76.776) (width 0.9) (layer F.Cu) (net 15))
 (segment (start 99.04199 81.046859) (end 102.762839 77.32601) (width 0.9) (layer F.Cu) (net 15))
 (segment (start 116.332 76.776) (end 116.332 74.676) (width 0.9) (layer F.Cu) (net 15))
 (segment (start 116.89002 119.106159) (end 116.89002 109.537148) (width 0.9) (layer F.Cu) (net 15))
 (segment (start 115.604168 120.392011) (end 116.89002 119.106159) (width 0.9) (layer F.Cu) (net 15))
 (segment (start 98.552 84.396) (end 98.552 82.296) (width 0.9) (layer F.Cu) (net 15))
 (segment (start 116.89002 109.537148) (end 96.584862 89.23199) (width 0.9) (layer F.Cu) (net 15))
 (segment (start 96.584862 89.23199) (end 96.584862 86.363138) (width 0.9) (layer F.Cu) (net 15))
 (segment (start 96.584862 86.363138) (end 98.552 84.396) (width 0.9) (layer F.Cu) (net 15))
 (segment (start 90.44461 124.46) (end 92.812589 122.092021) (width 0.9) (layer F.Cu) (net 20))
 (segment (start 92.812589 122.092021) (end 116.308335 122.092021) (width 0.9) (layer F.Cu) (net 20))
 (segment (start 78.232 124.46) (end 90.44461 124.46) (width 0.9) (layer F.Cu) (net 20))
 (segment (start 78.232 115.824) (end 78.232 124.46) (width 0.9) (layer B.Cu) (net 20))
 (via (at 78.232 124.46) (size 1.2) (drill 1) (layers F.Cu B.Cu) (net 20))
 (segment (start 85.344 112.776) (end 85.344 117.001002) (width 0.9) (layer F.Cu) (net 20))
 (segment (start 85.344 106.172) (end 85.344 112.776) (width 0.9) (layer F.Cu) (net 20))
 (segment (start 85.344 112.776) (end 81.28 112.776) (width 0.9) (layer F.Cu) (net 20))
 (segment (start 81.28 112.776) (end 78.232 115.824) (width 0.9) (layer F.Cu) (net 20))
 (via (at 78.232 115.824) (size 1.2) (drill 1) (layers F.Cu B.Cu) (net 20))
 (segment (start 85.344 117.001002) (end 88.262998 119.92) (width 0.9) (layer F.Cu) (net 20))
 (segment (start 88.262998 119.92) (end 88.453406 119.92) (width 0.9) (layer F.Cu) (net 20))
 (segment (start 88.453406 119.92) (end 89.408 119.92) (width 0.9) (layer F.Cu) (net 20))
 (segment (start 121.08001 54.159833) (end 121.08001 75.44799) (width 0.9) (layer F.Cu) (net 20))
 (segment (start 116.332 80.196) (end 116.332 82.296) (width 0.9) (layer F.Cu) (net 20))
 (segment (start 56.72 57.215821) (end 61.103821 52.832) (width 0.9) (layer F.Cu) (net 20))
 (segment (start 119.752177 52.832) (end 121.08001 54.159833) (width 0.9) (layer F.Cu) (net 20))
 (segment (start 58.42 74.676) (end 58.42 74.276) (width 0.9) (layer F.Cu) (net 20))
 (segment (start 58.42 74.276) (end 56.72 72.576) (width 0.9) (layer F.Cu) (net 20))
 (segment (start 56.72 72.576) (end 56.72 57.215821) (width 0.9) (layer F.Cu) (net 20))
 (segment (start 121.08001 75.44799) (end 116.332 80.196) (width 0.9) (layer F.Cu) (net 20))
 (segment (start 61.103821 52.832) (end 119.752177 52.832) (width 0.9) (layer F.Cu) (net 20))
 (segment (start 116.332 82.296) (end 118.032 82.296) (width 0.9) (layer F.Cu) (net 20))
 (segment (start 118.032 82.296) (end 118.59003 82.85403) (width 0.9) (layer F.Cu) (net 20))
 (segment (start 118.59003 82.85403) (end 118.59003 119.810326) (width 0.9) (layer F.Cu) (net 20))
 (segment (start 118.59003 119.810326) (end 116.308335 122.092021) (width 0.9) (layer F.Cu) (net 20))
 (segment (start 108.712 69.596) (end 94.488 69.596) (width 1.2) (layer B.Cu) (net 14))
 (segment (start 94.488 69.596) (end 87.884 76.2) (width 1.2) (layer B.Cu) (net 14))
 (segment (start 90.16399 109.97599) (end 96.012 115.824) (width 1.2) (layer B.Cu) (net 14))
 (segment (start 87.884 76.2) (end 90.16399 78.47999) (width 1.2) (layer B.Cu) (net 14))
 (segment (start 90.16399 78.47999) (end 90.16399 109.97599) (width 1.2) (layer B.Cu) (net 14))
 (segment (start 85.932 68.738126) (end 85.932 74.248) (width 1.2) (layer F.Cu) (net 14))
 (segment (start 85.932 74.248) (end 87.884 76.2) (width 1.2) (layer F.Cu) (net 14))
 (via (at 87.884 76.2) (size 1.2) (drill 1) (layers F.Cu B.Cu) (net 14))
 (segment (start 85.932 60.452) (end 85.932 68.738126) (width 1.2) (layer F.Cu) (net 14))
 (segment (start 85.932 68.738126) (end 77.194116 77.47601) (width 1.2) (layer F.Cu) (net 14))
 (segment (start 77.194116 77.47601) (end 68.44001 77.47601) (width 1.2) (layer F.Cu) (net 14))
 (segment (start 68.44001 77.47601) (end 66.04 75.076) (width 1.2) (layer F.Cu) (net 14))
 (segment (start 66.04 75.076) (end 66.04 74.676) (width 1.2) (layer F.Cu) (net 14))
 (segment (start 108.712 85.344) (end 108.712 82.296) (width 1.2) (layer F.Cu) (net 14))
 (segment (start 108.712 69.596) (end 108.712 85.344) (width 1.2) (layer B.Cu) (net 14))
 (via (at 108.712 85.344) (size 1.2) (drill 1) (layers F.Cu B.Cu) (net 14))
 (segment (start 108.712 74.676) (end 108.712 69.596) (width 1.2) (layer F.Cu) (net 14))
 (via (at 108.712 69.596) (size 1.2) (drill 1) (layers F.Cu B.Cu) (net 14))
 (segment (start 89.408 112.776) (end 89.408 117.644999) (width 1.2) (layer F.Cu) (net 14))
 (segment (start 89.408 100.853874) (end 89.408 112.776) (width 1.2) (layer F.Cu) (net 14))
 (segment (start 92.964 112.776) (end 96.012 115.824) (width 1.2) (layer F.Cu) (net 14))
 (segment (start 89.408 112.776) (end 92.964 112.776) (width 1.2) (layer F.Cu) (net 14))
 (via (at 96.012 115.824) (size 0.6) (drill 0.4) (layers F.Cu B.Cu) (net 14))
 (segment (start 92.964 98.552) (end 89.408 98.552) (width 1.2) (layer F.Cu) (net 14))
 (segment (start 89.408 98.552) (end 85.344 98.552) (width 1.2) (layer F.Cu) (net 14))
 (segment (start 89.408 100.853874) (end 89.408 98.552) (width 1.2) (layer F.Cu) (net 14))
 (segment (start 66.04 82.296) (end 66.04 74.676) (width 1.2) (layer F.Cu) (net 14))
 (segment (start 108.712 74.676) (end 106.172 74.676) (width 1.2) (layer F.Cu) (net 14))
 (segment (start 106.172 82.296) (end 108.712 82.296) (width 1.2) (layer F.Cu) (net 14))
 (segment (start 92.964 96.012) (end 92.964 98.552) (width 1.2) (layer F.Cu) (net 14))
 (segment (start 85.344 96.012) (end 85.344 98.552) (width 1.2) (layer F.Cu) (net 14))
 (segment (start 68.58 74.676) (end 66.04 74.676) (width 1.2) (layer F.Cu) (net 14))
 (segment (start 66.04 82.296) (end 68.58 82.296) (width 1.2) (layer F.Cu) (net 14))
 (segment (start 92.964 88.392) (end 92.964 83.928) (width 1.2) (layer F.Cu) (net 13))
 (segment (start 92.964 83.928) (end 91.332 82.296) (width 1.2) (layer F.Cu) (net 13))
 (segment (start 90.932 60.452) (end 90.932 69.056) (width 1.2) (layer F.Cu) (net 13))
 (segment (start 96.552 74.676) (end 98.552 74.676) (width 1.2) (layer F.Cu) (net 13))
 (segment (start 90.932 69.056) (end 96.552 74.676) (width 1.2) (layer F.Cu) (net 13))
 (segment (start 76.2 82.296) (end 91.332 82.296) (width 1.2) (layer F.Cu) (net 13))
 (segment (start 91.332 82.296) (end 98.552 75.076) (width 1.2) (layer F.Cu) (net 13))
 (segment (start 98.552 75.076) (end 98.552 74.676) (width 1.2) (layer F.Cu) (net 13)))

